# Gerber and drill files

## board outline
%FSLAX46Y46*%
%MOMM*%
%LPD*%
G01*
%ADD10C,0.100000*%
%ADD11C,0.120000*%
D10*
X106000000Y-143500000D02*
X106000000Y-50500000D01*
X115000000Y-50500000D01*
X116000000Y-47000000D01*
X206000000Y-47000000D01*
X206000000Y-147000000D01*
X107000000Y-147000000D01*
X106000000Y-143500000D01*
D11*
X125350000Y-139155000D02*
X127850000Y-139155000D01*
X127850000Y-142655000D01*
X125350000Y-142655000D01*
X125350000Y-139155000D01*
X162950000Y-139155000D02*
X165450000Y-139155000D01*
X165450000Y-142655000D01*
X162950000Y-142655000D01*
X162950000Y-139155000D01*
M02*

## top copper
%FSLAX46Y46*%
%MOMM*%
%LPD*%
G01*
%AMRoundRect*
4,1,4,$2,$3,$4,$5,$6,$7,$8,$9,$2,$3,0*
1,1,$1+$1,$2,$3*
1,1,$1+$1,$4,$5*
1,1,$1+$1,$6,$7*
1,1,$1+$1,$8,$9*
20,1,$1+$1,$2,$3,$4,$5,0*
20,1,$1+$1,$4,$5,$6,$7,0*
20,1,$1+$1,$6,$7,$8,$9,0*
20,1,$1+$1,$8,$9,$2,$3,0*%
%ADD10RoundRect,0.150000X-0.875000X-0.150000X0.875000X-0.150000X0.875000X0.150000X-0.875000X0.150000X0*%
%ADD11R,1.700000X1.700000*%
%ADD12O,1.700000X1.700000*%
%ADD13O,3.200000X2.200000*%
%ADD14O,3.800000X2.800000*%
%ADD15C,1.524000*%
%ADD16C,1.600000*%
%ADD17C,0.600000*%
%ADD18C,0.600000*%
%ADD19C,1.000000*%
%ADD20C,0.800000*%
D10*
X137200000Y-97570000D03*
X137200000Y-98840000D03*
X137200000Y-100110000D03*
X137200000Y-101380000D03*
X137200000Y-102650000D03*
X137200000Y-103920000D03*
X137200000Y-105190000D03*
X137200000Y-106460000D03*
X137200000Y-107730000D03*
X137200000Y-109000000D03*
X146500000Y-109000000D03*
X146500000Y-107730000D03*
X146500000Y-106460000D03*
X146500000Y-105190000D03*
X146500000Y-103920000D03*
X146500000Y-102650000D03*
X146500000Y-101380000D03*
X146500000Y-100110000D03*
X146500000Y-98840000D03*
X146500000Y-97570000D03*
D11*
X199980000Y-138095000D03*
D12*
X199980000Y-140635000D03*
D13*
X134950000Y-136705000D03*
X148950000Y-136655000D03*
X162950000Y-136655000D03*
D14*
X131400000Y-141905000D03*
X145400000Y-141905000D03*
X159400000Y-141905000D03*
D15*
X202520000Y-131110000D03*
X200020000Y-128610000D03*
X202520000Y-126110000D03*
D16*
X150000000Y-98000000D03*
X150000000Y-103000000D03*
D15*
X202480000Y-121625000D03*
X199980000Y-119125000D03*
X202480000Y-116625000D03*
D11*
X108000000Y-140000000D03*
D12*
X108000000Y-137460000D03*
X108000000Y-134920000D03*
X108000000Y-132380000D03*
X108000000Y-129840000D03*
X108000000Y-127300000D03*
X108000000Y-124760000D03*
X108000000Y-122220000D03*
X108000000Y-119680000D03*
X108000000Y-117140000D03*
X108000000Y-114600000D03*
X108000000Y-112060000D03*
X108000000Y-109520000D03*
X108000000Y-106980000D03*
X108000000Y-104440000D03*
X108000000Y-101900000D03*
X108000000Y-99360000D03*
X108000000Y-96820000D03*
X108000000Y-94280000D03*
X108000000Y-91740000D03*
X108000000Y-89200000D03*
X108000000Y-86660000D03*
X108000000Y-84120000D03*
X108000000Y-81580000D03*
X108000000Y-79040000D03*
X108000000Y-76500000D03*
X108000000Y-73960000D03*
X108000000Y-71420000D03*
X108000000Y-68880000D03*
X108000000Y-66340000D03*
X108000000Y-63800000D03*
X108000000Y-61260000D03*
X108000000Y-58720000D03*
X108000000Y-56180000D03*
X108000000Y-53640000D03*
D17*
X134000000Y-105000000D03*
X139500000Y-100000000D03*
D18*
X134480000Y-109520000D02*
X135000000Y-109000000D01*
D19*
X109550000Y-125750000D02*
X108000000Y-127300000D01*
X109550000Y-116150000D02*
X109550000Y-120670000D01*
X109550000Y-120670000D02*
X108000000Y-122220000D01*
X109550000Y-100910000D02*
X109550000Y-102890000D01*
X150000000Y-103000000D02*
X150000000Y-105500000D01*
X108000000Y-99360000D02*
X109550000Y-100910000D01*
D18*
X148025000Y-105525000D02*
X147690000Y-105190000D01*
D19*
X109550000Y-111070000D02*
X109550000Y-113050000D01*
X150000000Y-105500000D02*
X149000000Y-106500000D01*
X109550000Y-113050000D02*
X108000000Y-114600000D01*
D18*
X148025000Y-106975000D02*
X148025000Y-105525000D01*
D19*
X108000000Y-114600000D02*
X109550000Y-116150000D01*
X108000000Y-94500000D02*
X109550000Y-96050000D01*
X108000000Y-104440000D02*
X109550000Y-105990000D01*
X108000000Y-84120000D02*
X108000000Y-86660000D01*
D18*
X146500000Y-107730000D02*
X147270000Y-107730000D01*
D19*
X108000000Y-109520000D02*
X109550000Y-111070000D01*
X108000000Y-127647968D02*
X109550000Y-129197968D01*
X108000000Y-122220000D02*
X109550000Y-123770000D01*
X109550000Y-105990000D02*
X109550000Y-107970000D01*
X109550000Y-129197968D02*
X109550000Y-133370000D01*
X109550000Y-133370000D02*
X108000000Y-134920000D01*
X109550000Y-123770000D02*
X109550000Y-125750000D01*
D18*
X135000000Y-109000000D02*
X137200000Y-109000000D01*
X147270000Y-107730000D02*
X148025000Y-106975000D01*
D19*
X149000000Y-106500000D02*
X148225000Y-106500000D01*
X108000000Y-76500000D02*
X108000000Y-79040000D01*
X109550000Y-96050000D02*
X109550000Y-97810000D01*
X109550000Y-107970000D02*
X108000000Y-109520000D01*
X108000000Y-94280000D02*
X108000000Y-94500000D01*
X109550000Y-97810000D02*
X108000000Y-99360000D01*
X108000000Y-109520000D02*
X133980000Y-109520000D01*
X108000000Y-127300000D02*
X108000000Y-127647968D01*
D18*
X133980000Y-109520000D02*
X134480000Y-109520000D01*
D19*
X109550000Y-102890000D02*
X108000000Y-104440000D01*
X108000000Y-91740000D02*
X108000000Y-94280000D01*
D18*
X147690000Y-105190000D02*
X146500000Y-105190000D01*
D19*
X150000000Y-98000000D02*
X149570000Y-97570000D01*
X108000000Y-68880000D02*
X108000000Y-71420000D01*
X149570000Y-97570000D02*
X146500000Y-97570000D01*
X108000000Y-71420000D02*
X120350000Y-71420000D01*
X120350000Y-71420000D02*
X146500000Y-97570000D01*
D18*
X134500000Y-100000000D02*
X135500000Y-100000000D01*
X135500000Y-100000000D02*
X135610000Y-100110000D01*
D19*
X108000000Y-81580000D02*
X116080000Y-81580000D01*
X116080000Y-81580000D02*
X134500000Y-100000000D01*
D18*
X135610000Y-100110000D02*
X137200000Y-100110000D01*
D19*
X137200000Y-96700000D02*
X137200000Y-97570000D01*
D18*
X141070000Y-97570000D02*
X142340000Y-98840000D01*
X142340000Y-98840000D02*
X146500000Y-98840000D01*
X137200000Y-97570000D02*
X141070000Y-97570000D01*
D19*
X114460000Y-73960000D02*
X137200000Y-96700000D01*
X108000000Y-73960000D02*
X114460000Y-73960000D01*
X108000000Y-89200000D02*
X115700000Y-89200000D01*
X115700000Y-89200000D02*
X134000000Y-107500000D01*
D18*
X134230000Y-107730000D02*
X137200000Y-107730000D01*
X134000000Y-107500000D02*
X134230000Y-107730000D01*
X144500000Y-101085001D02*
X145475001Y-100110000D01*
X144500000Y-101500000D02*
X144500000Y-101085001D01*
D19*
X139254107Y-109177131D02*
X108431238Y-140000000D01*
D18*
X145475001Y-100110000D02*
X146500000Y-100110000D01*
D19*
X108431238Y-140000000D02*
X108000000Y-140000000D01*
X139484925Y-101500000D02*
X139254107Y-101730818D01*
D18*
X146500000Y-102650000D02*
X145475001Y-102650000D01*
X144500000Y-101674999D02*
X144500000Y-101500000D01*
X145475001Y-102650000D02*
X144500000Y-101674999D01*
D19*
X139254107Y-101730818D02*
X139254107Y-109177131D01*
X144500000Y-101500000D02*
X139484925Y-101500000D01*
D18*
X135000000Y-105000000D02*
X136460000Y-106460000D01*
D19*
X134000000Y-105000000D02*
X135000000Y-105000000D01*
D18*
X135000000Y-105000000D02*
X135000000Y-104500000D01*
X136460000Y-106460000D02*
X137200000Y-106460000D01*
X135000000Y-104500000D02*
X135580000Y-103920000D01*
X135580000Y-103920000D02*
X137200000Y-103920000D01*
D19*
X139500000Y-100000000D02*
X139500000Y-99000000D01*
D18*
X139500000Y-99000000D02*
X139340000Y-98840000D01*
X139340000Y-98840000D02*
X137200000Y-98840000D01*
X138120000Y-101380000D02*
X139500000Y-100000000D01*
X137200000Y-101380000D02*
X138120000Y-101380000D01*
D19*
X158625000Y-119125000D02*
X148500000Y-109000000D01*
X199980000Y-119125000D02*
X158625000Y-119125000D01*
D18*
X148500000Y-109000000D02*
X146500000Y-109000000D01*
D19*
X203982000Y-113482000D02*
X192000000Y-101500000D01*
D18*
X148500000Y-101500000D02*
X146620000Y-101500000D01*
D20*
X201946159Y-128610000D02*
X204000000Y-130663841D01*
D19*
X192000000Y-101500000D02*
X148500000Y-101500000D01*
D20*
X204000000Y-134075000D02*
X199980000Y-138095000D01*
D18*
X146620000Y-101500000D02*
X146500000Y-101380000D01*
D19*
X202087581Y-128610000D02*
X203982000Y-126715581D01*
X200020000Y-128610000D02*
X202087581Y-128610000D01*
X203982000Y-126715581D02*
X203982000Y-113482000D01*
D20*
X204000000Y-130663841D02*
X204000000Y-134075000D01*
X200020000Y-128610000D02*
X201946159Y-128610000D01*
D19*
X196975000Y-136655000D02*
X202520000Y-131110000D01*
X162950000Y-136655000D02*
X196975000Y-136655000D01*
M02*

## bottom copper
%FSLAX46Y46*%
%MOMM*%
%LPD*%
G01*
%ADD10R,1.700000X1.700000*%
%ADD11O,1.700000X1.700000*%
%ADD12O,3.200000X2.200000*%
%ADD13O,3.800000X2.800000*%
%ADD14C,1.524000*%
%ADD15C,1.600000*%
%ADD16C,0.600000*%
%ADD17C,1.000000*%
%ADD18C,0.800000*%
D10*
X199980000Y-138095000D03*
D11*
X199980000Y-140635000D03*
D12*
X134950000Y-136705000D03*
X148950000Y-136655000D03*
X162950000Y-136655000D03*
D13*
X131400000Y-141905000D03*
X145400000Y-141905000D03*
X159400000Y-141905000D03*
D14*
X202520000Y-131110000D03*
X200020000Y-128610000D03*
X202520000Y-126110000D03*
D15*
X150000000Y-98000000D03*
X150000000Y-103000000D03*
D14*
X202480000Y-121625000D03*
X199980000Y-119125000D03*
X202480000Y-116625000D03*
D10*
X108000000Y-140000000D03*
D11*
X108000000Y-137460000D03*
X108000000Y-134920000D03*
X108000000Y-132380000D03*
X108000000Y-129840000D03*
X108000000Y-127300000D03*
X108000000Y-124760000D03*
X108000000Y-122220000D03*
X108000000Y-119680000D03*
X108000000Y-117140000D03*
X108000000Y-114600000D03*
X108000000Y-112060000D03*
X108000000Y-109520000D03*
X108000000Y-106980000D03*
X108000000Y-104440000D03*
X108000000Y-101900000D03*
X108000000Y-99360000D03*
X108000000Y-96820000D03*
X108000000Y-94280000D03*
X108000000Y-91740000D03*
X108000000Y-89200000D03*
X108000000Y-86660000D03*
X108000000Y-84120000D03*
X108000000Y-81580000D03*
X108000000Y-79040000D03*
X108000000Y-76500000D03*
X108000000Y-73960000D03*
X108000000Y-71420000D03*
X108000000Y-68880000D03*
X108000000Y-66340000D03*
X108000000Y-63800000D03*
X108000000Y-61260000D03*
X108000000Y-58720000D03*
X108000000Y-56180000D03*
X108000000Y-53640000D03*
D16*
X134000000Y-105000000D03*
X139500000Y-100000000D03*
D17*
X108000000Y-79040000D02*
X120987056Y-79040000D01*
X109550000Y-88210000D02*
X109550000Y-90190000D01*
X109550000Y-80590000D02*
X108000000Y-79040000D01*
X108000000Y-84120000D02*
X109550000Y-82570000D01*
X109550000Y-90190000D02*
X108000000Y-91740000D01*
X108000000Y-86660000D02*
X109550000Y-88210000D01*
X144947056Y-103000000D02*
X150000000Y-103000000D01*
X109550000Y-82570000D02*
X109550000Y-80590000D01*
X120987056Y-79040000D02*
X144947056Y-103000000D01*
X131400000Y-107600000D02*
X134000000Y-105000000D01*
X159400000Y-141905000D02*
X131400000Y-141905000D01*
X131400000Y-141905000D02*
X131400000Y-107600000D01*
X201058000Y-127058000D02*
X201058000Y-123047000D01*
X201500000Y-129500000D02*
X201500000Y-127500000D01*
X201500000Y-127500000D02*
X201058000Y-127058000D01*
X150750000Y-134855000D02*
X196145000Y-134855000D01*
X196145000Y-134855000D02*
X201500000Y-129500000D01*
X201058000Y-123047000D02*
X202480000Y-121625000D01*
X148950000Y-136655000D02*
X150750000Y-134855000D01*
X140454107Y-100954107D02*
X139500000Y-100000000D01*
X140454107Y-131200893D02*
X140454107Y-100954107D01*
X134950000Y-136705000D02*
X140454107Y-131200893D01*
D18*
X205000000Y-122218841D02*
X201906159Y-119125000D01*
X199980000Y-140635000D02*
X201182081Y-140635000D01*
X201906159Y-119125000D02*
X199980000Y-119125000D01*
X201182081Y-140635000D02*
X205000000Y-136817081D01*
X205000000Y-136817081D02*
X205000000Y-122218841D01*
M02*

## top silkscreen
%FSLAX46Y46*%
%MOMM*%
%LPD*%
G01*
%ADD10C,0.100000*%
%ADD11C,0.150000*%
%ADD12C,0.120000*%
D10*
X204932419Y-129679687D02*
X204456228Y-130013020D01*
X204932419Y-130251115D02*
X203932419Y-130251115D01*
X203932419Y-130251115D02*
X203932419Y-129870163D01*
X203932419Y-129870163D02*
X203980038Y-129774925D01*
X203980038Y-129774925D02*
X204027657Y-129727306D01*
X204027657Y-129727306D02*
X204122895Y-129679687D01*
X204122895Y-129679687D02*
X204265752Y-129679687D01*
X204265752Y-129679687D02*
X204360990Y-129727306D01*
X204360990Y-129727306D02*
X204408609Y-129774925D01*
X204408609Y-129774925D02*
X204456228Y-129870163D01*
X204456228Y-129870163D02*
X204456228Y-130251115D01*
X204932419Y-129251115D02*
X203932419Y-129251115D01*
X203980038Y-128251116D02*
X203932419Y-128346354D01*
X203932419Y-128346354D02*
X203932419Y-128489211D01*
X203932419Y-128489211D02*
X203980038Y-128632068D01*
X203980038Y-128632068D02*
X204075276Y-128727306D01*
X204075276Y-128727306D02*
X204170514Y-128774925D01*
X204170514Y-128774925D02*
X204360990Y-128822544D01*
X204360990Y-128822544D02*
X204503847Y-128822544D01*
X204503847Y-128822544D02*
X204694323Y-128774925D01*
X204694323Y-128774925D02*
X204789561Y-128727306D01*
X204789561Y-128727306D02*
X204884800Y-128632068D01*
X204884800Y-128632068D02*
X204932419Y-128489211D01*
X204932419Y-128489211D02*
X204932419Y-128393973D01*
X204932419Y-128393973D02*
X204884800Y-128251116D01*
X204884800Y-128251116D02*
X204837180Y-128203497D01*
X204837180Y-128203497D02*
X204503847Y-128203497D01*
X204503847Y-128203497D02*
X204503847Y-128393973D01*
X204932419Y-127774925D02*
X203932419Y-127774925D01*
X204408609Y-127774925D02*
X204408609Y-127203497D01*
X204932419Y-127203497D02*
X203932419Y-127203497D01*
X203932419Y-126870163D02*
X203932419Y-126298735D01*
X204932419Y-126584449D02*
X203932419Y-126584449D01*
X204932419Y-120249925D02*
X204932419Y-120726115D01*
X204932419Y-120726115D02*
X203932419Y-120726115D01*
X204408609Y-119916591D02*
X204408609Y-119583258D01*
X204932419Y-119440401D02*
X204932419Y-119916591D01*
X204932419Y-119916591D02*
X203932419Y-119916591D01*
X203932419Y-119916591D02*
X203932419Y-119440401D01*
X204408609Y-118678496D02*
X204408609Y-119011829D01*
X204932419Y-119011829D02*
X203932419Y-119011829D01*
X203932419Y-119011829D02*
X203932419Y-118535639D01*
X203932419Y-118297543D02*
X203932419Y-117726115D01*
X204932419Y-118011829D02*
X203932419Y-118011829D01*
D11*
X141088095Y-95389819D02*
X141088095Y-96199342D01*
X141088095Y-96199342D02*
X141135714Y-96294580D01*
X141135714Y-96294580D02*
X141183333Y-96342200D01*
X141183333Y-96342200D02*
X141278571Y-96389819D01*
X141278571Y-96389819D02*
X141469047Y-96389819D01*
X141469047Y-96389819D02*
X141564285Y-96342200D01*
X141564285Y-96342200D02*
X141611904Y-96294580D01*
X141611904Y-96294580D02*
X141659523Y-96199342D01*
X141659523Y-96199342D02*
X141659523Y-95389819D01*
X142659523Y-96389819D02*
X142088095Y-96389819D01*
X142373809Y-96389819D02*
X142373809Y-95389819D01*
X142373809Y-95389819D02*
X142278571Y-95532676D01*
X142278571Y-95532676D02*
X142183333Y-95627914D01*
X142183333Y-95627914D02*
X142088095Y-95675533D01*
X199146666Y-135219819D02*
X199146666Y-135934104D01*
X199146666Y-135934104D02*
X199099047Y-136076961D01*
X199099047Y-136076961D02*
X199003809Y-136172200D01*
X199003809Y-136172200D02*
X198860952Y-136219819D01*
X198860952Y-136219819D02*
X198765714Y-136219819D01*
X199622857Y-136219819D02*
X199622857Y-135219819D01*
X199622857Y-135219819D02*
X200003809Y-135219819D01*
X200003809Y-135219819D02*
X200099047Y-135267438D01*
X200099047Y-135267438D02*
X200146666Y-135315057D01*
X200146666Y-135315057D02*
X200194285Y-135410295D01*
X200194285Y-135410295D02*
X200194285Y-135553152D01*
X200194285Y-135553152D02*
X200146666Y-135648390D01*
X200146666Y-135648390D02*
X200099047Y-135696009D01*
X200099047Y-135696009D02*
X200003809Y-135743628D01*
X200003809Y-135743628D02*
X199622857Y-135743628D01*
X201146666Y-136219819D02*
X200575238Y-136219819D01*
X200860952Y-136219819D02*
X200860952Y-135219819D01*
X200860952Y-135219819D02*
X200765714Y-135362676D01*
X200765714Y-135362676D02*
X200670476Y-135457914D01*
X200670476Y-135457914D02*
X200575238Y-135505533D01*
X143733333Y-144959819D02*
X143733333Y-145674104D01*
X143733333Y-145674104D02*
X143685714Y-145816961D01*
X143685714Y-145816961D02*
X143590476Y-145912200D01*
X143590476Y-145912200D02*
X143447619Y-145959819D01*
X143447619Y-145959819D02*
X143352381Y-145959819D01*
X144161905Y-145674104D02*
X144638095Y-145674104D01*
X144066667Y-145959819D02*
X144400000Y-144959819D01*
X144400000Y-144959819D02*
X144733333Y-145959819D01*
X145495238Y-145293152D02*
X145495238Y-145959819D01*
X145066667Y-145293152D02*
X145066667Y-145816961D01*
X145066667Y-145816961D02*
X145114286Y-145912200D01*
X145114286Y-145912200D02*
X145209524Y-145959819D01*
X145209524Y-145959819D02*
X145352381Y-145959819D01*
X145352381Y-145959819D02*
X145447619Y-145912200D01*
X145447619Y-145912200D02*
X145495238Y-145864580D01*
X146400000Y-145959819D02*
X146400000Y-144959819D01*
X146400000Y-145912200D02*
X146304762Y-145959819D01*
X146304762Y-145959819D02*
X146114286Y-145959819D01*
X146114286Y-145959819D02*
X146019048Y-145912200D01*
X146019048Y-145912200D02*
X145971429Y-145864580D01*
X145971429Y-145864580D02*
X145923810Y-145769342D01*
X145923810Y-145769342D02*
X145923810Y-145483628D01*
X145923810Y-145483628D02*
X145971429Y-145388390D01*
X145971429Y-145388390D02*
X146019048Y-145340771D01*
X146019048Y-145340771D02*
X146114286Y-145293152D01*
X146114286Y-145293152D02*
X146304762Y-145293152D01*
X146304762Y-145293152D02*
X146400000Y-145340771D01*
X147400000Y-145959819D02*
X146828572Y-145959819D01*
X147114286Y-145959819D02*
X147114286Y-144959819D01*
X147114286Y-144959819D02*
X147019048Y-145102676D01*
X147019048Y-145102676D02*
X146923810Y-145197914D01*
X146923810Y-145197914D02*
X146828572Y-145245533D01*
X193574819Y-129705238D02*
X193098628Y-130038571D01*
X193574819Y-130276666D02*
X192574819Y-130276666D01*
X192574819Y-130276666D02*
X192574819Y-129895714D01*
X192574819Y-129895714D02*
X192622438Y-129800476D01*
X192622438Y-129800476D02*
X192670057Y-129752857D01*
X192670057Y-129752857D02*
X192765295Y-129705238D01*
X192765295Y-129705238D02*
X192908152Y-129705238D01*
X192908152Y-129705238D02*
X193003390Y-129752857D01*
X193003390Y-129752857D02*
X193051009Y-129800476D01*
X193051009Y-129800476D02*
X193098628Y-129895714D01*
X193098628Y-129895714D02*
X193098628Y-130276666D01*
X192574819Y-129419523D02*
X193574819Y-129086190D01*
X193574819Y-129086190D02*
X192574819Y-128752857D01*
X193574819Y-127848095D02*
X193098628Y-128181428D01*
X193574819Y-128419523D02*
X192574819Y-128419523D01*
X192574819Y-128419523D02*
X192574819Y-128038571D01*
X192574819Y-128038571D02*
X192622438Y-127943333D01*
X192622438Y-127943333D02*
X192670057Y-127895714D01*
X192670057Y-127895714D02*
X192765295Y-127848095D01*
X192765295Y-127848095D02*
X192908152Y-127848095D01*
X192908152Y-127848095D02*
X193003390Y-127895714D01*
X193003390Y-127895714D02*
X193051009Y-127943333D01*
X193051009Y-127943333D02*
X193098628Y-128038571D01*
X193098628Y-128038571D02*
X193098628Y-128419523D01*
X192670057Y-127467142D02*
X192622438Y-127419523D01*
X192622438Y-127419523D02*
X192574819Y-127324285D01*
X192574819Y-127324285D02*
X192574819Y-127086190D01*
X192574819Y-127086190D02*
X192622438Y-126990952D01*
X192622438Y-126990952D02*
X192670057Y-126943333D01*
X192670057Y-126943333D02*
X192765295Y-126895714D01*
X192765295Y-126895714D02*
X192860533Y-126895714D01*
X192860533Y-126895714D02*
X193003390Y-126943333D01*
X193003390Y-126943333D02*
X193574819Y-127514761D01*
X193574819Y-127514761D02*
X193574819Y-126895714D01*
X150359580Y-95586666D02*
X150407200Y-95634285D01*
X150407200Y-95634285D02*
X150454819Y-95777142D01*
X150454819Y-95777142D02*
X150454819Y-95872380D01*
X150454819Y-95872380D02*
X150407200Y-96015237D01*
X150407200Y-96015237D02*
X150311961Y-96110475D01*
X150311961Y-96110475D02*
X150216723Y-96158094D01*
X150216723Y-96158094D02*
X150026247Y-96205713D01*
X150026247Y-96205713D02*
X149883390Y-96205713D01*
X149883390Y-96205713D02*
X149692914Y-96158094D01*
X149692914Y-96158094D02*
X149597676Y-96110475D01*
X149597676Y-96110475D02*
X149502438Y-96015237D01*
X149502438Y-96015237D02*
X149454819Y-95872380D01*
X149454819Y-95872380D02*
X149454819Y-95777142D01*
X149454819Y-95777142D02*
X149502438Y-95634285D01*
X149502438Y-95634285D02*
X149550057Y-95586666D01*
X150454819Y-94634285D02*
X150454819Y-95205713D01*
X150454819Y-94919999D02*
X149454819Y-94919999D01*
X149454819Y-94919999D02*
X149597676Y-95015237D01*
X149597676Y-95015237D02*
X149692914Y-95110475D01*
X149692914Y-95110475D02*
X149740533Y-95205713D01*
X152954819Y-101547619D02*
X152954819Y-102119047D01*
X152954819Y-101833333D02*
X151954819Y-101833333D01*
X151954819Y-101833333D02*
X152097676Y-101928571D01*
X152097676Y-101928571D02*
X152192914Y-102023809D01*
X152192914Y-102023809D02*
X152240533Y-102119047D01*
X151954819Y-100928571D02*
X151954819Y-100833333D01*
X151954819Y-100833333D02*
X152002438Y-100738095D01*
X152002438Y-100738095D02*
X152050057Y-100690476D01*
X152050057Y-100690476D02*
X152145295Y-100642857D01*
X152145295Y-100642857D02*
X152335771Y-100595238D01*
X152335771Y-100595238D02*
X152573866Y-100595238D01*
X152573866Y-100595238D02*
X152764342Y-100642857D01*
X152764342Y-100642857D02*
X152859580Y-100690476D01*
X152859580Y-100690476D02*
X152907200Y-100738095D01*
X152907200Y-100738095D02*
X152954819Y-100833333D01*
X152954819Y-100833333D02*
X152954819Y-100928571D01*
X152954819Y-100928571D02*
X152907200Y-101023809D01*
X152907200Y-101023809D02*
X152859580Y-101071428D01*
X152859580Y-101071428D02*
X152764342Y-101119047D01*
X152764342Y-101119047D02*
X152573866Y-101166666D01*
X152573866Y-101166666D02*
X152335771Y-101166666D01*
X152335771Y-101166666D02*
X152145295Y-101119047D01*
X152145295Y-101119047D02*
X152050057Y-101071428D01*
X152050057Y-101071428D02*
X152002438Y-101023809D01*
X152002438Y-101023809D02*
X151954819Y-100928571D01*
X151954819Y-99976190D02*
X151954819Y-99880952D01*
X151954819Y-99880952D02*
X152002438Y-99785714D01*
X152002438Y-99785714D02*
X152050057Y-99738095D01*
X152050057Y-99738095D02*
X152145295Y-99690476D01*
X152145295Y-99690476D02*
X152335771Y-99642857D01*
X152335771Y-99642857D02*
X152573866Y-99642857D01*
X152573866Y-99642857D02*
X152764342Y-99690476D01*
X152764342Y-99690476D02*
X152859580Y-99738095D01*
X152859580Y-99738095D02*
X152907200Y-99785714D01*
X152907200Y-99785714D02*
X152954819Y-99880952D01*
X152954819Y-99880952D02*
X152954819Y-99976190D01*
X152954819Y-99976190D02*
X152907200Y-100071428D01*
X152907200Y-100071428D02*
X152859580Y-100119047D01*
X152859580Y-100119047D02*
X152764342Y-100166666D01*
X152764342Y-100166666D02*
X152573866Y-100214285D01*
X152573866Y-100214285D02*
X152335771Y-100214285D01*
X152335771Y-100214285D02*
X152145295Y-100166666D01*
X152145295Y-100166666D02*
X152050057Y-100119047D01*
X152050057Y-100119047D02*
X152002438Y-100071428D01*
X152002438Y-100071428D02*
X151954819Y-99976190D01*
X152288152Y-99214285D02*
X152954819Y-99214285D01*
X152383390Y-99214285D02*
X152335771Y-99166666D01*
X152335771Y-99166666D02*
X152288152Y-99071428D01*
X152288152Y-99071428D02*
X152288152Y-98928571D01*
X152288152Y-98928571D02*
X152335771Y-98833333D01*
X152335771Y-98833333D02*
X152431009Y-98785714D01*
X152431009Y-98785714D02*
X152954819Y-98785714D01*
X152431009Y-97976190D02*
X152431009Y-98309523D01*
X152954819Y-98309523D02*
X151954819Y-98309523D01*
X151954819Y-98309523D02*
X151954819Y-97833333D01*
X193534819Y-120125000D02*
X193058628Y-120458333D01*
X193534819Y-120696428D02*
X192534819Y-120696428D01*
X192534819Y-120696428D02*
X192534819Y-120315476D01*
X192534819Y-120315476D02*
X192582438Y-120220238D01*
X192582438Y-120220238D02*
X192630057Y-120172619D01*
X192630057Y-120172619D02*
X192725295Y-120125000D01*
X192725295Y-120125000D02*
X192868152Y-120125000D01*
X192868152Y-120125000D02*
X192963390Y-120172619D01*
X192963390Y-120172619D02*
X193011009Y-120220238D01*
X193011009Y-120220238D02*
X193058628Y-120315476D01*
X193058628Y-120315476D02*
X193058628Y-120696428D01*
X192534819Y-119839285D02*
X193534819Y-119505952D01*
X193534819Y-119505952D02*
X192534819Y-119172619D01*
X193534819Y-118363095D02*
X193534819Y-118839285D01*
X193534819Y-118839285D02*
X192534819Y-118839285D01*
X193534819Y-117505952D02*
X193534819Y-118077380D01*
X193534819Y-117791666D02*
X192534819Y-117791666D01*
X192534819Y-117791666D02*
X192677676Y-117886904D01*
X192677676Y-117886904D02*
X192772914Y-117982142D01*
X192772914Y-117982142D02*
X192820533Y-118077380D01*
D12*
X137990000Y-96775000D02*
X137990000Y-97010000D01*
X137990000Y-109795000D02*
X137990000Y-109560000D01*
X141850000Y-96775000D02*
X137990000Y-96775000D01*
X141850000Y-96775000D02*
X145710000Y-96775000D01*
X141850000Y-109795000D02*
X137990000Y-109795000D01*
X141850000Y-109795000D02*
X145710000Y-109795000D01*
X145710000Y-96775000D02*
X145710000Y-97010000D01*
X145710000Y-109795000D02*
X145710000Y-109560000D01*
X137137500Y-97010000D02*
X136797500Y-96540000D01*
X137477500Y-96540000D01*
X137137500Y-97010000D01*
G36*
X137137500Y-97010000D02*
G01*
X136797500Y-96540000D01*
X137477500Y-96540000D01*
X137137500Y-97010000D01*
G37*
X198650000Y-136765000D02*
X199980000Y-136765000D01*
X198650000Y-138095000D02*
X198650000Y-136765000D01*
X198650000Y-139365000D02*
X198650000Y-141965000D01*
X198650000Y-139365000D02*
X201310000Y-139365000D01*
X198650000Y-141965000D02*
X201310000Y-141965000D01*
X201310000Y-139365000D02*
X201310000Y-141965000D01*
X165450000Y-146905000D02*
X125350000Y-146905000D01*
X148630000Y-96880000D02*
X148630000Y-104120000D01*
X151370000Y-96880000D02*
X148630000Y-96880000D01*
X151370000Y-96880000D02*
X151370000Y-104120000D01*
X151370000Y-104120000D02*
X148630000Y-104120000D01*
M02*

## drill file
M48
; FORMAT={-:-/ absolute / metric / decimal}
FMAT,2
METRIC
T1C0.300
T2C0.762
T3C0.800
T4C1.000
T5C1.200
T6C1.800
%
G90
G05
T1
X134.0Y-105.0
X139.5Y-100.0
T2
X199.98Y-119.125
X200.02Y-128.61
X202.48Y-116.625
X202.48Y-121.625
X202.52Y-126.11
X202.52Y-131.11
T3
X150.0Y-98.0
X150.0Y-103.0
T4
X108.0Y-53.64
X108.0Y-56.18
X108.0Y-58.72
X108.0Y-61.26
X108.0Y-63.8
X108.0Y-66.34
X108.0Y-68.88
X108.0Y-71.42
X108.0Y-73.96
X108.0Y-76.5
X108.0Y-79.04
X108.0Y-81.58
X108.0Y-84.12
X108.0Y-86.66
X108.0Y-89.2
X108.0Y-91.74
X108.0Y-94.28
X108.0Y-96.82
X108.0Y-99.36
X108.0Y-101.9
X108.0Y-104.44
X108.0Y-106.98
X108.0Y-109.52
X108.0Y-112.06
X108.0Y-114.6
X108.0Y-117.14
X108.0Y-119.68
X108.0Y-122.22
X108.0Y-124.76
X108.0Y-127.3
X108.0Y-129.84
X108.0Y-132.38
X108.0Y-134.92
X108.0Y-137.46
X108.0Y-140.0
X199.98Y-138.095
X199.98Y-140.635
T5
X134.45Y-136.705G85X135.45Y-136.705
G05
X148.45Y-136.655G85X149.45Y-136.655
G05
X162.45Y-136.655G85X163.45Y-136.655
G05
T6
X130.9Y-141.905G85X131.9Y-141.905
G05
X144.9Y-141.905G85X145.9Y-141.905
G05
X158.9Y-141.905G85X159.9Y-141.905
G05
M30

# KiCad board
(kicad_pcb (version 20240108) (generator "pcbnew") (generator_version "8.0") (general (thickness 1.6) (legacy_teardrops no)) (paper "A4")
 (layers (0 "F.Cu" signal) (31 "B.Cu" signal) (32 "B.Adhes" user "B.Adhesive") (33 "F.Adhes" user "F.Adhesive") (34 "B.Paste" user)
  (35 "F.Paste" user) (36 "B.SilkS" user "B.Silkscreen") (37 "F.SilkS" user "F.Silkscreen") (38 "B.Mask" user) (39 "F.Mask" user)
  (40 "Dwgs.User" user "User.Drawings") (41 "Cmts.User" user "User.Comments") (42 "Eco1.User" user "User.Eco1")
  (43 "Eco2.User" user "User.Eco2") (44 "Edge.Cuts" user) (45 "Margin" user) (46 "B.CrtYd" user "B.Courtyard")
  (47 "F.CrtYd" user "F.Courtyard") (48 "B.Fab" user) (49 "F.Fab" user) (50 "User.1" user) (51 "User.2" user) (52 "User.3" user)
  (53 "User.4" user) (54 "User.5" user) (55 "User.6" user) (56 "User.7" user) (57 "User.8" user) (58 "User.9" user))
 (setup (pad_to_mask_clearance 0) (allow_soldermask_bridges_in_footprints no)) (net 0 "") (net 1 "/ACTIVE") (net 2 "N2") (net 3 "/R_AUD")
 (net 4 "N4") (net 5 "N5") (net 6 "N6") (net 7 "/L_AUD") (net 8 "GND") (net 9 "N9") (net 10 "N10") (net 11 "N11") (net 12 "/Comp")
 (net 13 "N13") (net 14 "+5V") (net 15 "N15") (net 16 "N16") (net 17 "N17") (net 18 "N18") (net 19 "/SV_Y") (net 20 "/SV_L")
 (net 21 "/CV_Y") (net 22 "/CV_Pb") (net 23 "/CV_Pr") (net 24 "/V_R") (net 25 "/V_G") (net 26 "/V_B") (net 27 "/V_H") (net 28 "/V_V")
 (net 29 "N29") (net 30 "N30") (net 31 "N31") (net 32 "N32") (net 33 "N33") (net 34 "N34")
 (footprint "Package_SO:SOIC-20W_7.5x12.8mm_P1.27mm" (layer "F.Cu") (at 141.85 103.285)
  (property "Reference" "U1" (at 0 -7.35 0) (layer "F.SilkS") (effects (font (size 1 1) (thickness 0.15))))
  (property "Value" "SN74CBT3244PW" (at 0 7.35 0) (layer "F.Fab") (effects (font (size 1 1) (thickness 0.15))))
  (fp_line (start -3.86 -6.51) (end -3.86 -6.275) (stroke (width 0.12) (type solid)) (layer "F.SilkS"))
  (fp_line (start -3.86 6.51) (end -3.86 6.275) (stroke (width 0.12) (type solid)) (layer "F.SilkS"))
  (fp_line (start 0 -6.51) (end -3.86 -6.51) (stroke (width 0.12) (type solid)) (layer "F.SilkS"))
  (fp_line (start 0 -6.51) (end 3.86 -6.51) (stroke (width 0.12) (type solid)) (layer "F.SilkS"))
  (fp_line (start 0 6.51) (end -3.86 6.51) (stroke (width 0.12) (type solid)) (layer "F.SilkS"))
  (fp_line (start 0 6.51) (end 3.86 6.51) (stroke (width 0.12) (type solid)) (layer "F.SilkS"))
  (fp_line (start 3.86 -6.51) (end 3.86 -6.275) (stroke (width 0.12) (type solid)) (layer "F.SilkS"))
  (fp_line (start 3.86 6.51) (end 3.86 6.275) (stroke (width 0.12) (type solid)) (layer "F.SilkS"))
  (fp_poly
   (pts (xy -4.7125 -6.275) (xy -5.0525 -6.745) (xy -4.3725 -6.745) (xy -4.7125 -6.275)) (stroke (width 0.12) (type solid)) (fill solid)
   (layer "F.SilkS"))
  (pad "1" smd roundrect (at -4.65 -5.715) (size 2.05 0.6) (layers "F.Cu" "F.Paste" "F.Mask") (roundrect_rratio 0.25) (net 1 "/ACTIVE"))
  (pad "2" smd roundrect (at -4.65 -4.445) (size 2.05 0.6) (layers "F.Cu" "F.Paste" "F.Mask") (roundrect_rratio 0.25) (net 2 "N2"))
  (pad "3" smd roundrect (at -4.65 -3.175) (size 2.05 0.6) (layers "F.Cu" "F.Paste" "F.Mask") (roundrect_rratio 0.25) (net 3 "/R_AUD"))
  (pad "4" smd roundrect (at -4.65 -1.905) (size 2.05 0.6) (layers "F.Cu" "F.Paste" "F.Mask") (roundrect_rratio 0.25) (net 2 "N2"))
  (pad "5" smd roundrect (at -4.65 -0.635) (size 2.05 0.6) (layers "F.Cu" "F.Paste" "F.Mask") (roundrect_rratio 0.25) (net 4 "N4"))
  (pad "6" smd roundrect (at -4.65 0.635) (size 2.05 0.6) (layers "F.Cu" "F.Paste" "F.Mask") (roundrect_rratio 0.25) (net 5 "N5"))
  (pad "7" smd roundrect (at -4.65 1.905) (size 2.05 0.6) (layers "F.Cu" "F.Paste" "F.Mask") (roundrect_rratio 0.25) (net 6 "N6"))
  (pad "8" smd roundrect (at -4.65 3.175) (size 2.05 0.6) (layers "F.Cu" "F.Paste" "F.Mask") (roundrect_rratio 0.25) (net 5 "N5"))
  (pad "9" smd roundrect (at -4.65 4.445) (size 2.05 0.6) (layers "F.Cu" "F.Paste" "F.Mask") (roundrect_rratio 0.25) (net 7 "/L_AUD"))
  (pad "10" smd roundrect (at -4.65 5.715) (size 2.05 0.6) (layers "F.Cu" "F.Paste" "F.Mask") (roundrect_rratio 0.25) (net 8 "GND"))
  (pad "11" smd roundrect (at 4.65 5.715) (size 2.05 0.6) (layers "F.Cu" "F.Paste" "F.Mask") (roundrect_rratio 0.25) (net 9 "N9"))
  (pad "12" smd roundrect (at 4.65 4.445) (size 2.05 0.6) (layers "F.Cu" "F.Paste" "F.Mask") (roundrect_rratio 0.25) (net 8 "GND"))
  (pad "13" smd roundrect (at 4.65 3.175) (size 2.05 0.6) (layers "F.Cu" "F.Paste" "F.Mask") (roundrect_rratio 0.25) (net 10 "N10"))
  (pad "14" smd roundrect (at 4.65 1.905) (size 2.05 0.6) (layers "F.Cu" "F.Paste" "F.Mask") (roundrect_rratio 0.25) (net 8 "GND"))
  (pad "15" smd roundrect (at 4.65 0.635) (size 2.05 0.6) (layers "F.Cu" "F.Paste" "F.Mask") (roundrect_rratio 0.25) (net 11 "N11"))
  (pad "16" smd roundrect (at 4.65 -0.635) (size 2.05 0.6) (layers "F.Cu" "F.Paste" "F.Mask") (roundrect_rratio 0.25) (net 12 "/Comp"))
  (pad "17" smd roundrect (at 4.65 -1.905) (size 2.05 0.6) (layers "F.Cu" "F.Paste" "F.Mask") (roundrect_rratio 0.25) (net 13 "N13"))
  (pad "18" smd roundrect (at 4.65 -3.175) (size 2.05 0.6) (layers "F.Cu" "F.Paste" "F.Mask") (roundrect_rratio 0.25) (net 12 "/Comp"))
  (pad "19" smd roundrect (at 4.65 -4.445) (size 2.05 0.6) (layers "F.Cu" "F.Paste" "F.Mask") (roundrect_rratio 0.25) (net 1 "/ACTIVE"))
  (pad "20" smd roundrect (at 4.65 -5.715) (size 2.05 0.6) (layers "F.Cu" "F.Paste" "F.Mask") (roundrect_rratio 0.25) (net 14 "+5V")))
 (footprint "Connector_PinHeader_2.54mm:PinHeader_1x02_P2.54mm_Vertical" (layer "F.Cu") (at 199.98 138.095)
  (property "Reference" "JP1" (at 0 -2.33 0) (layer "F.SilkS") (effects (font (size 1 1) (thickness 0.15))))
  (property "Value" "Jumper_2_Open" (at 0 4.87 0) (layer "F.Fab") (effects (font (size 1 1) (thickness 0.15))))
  (fp_line (start -1.33 -1.33) (end 0 -1.33) (stroke (width 0.12) (type solid)) (layer "F.SilkS"))
  (fp_line (start -1.33 0) (end -1.33 -1.33) (stroke (width 0.12) (type solid)) (layer "F.SilkS"))
  (fp_line (start -1.33 1.27) (end -1.33 3.87) (stroke (width 0.12) (type solid)) (layer "F.SilkS"))
  (fp_line (start -1.33 1.27) (end 1.33 1.27) (stroke (width 0.12) (type solid)) (layer "F.SilkS"))
  (fp_line (start -1.33 3.87) (end 1.33 3.87) (stroke (width 0.12) (type solid)) (layer "F.SilkS"))
  (fp_line (start 1.33 1.27) (end 1.33 3.87) (stroke (width 0.12) (type solid)) (layer "F.SilkS"))
  (pad "1" thru_hole rect (at 0 0) (size 1.7 1.7) (drill 1) (layers "*.Cu" "*.Mask") (remove_unused_layers no) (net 13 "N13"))
  (pad "2" thru_hole oval (at 0 2.54) (size 1.7 1.7) (drill 1) (layers "*.Cu" "*.Mask") (remove_unused_layers no) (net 9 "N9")))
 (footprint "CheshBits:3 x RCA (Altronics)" (layer "F.Cu") (at 145.4 146.905)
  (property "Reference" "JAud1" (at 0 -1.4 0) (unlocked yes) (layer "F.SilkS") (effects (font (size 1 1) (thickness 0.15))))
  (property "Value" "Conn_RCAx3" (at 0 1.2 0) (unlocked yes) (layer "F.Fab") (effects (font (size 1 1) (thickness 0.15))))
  (fp_line (start 20.05 0) (end -20.05 0) (stroke (width 0.12) (type default)) (layer "F.SilkS"))
  (fp_rect (start -20.05 -7.75) (end -17.55 -4.25) (stroke (width 0.12) (type default)) (fill none) (layer "Edge.Cuts"))
  (fp_rect (start 17.55 -7.75) (end 20.05 -4.25) (stroke (width 0.12) (type default)) (fill none) (layer "Edge.Cuts"))
  (pad "1" thru_hole oval (at -10.45 -10.2) (size 3.2 2.2) (drill oval 2.2 1.2) (layers "*.Cu" "*.Mask") (remove_unused_layers no)
   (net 2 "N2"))
  (pad "2" thru_hole oval (at 3.55 -10.25) (size 3.2 2.2) (drill oval 2.2 1.2) (layers "*.Cu" "*.Mask") (remove_unused_layers no)
   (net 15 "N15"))
  (pad "3" thru_hole oval (at 17.55 -10.25) (size 3.2 2.2) (drill oval 2.2 1.2) (layers "*.Cu" "*.Mask") (remove_unused_layers no)
   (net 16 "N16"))
  (pad "4" thru_hole oval (at -14 -5) (size 3.8 2.8) (drill oval 2.8 1.8) (layers "*.Cu" "*.Mask") (remove_unused_layers no) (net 5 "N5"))
  (pad "4" thru_hole oval (at 0 -5) (size 3.8 2.8) (drill oval 2.8 1.8) (layers "*.Cu" "*.Mask") (remove_unused_layers no) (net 5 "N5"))
  (pad "4" thru_hole oval (at 14 -5) (size 3.8 2.8) (drill oval 2.8 1.8) (layers "*.Cu" "*.Mask") (remove_unused_layers no) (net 5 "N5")))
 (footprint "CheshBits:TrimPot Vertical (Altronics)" (layer "F.Cu") (at 193.62 128.61 90)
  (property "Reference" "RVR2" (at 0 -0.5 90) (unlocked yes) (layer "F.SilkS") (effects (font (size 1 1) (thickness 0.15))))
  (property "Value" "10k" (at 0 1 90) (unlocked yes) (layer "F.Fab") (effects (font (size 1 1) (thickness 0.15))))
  (pad "1" thru_hole circle (at -2.5 8.9 90) (size 1.524 1.524) (drill 0.762) (layers "*.Cu" "*.Mask") (remove_unused_layers no)
   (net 16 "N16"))
  (pad "2" thru_hole circle (at 0 6.4 90) (size 1.524 1.524) (drill 0.762) (layers "*.Cu" "*.Mask") (remove_unused_layers no) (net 13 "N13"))
  (pad "3" thru_hole circle (at 2.5 8.9 90) (size 1.524 1.524) (drill 0.762) (layers "*.Cu" "*.Mask") (remove_unused_layers no)
   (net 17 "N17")))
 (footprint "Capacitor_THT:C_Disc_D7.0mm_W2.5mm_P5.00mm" (layer "F.Cu") (at 150 98 -90)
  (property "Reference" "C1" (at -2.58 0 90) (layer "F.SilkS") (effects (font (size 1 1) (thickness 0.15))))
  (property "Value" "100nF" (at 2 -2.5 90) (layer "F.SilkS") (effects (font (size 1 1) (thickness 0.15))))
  (fp_line (start -1.12 1.37) (end 6.12 1.37) (stroke (width 0.12) (type solid)) (layer "F.SilkS"))
  (fp_line (start -1.12 -1.37) (end -1.12 1.37) (stroke (width 0.12) (type solid)) (layer "F.SilkS"))
  (fp_line (start -1.12 -1.37) (end 6.12 -1.37) (stroke (width 0.12) (type solid)) (layer "F.SilkS"))
  (fp_line (start 6.12 -1.37) (end 6.12 1.37) (stroke (width 0.12) (type solid)) (layer "F.SilkS"))
  (pad "1" thru_hole circle (at 0 0 270) (size 1.6 1.6) (drill 0.8) (layers "*.Cu" "*.Mask") (remove_unused_layers no) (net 14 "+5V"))
  (pad "2" thru_hole circle (at 5 0 270) (size 1.6 1.6) (drill 0.8) (layers "*.Cu" "*.Mask") (remove_unused_layers no) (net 8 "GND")))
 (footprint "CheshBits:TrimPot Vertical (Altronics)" (layer "F.Cu") (at 193.58 119.125 90)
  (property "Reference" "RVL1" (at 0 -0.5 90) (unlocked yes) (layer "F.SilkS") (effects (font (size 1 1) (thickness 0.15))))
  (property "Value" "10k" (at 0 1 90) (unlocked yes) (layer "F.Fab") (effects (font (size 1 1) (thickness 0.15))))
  (pad "1" thru_hole circle (at -2.5 8.9 90) (size 1.524 1.524) (drill 0.762) (layers "*.Cu" "*.Mask") (remove_unused_layers no)
   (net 15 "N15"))
  (pad "2" thru_hole circle (at 0 6.4 90) (size 1.524 1.524) (drill 0.762) (layers "*.Cu" "*.Mask") (remove_unused_layers no) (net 9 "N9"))
  (pad "3" thru_hole circle (at 2.5 8.9 90) (size 1.524 1.524) (drill 0.762) (layers "*.Cu" "*.Mask") (remove_unused_layers no)
   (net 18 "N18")))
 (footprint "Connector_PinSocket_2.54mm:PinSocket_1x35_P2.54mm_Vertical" (layer "B.Cu") (at 108 140)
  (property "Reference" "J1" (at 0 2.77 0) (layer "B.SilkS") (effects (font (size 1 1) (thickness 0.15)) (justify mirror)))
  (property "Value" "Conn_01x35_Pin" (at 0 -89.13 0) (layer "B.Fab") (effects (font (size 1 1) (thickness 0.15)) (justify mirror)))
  (pad "1" thru_hole rect (at 0 0) (size 1.7 1.7) (drill 1) (layers "*.Cu" "*.Mask") (remove_unused_layers no) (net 12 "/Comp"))
  (pad "2" thru_hole oval (at 0 -2.54) (size 1.7 1.7) (drill 1) (layers "*.Cu" "*.Mask") (remove_unused_layers no) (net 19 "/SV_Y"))
  (pad "3" thru_hole oval (at 0 -5.08) (size 1.7 1.7) (drill 1) (layers "*.Cu" "*.Mask") (remove_unused_layers no) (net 8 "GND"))
  (pad "4" thru_hole oval (at 0 -7.62) (size 1.7 1.7) (drill 1) (layers "*.Cu" "*.Mask") (remove_unused_layers no) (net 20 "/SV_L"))
  (pad "5" thru_hole oval (at 0 -10.16) (size 1.7 1.7) (drill 1) (layers "*.Cu" "*.Mask") (remove_unused_layers no) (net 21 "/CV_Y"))
  (pad "6" thru_hole oval (at 0 -12.7) (size 1.7 1.7) (drill 1) (layers "*.Cu" "*.Mask") (remove_unused_layers no) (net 8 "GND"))
  (pad "7" thru_hole oval (at 0 -15.24) (size 1.7 1.7) (drill 1) (layers "*.Cu" "*.Mask") (remove_unused_layers no) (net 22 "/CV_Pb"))
  (pad "8" thru_hole oval (at 0 -17.78) (size 1.7 1.7) (drill 1) (layers "*.Cu" "*.Mask") (remove_unused_layers no) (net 8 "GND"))
  (pad "9" thru_hole oval (at 0 -20.32) (size 1.7 1.7) (drill 1) (layers "*.Cu" "*.Mask") (remove_unused_layers no) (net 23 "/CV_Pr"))
  (pad "10" thru_hole oval (at 0 -22.86) (size 1.7 1.7) (drill 1) (layers "*.Cu" "*.Mask") (remove_unused_layers no) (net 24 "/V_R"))
  (pad "11" thru_hole oval (at 0 -25.4) (size 1.7 1.7) (drill 1) (layers "*.Cu" "*.Mask") (remove_unused_layers no) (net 8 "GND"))
  (pad "12" thru_hole oval (at 0 -27.94) (size 1.7 1.7) (drill 1) (layers "*.Cu" "*.Mask") (remove_unused_layers no) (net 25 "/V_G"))
  (pad "13" thru_hole oval (at 0 -30.48) (size 1.7 1.7) (drill 1) (layers "*.Cu" "*.Mask") (remove_unused_layers no) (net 8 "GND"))
  (pad "14" thru_hole oval (at 0 -33.02) (size 1.7 1.7) (drill 1) (layers "*.Cu" "*.Mask") (remove_unused_layers no) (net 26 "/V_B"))
  (pad "15" thru_hole oval (at 0 -35.56) (size 1.7 1.7) (drill 1) (layers "*.Cu" "*.Mask") (remove_unused_layers no) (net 8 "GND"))
  (pad "16" thru_hole oval (at 0 -38.1) (size 1.7 1.7) (drill 1) (layers "*.Cu" "*.Mask") (remove_unused_layers no) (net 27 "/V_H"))
  (pad "17" thru_hole oval (at 0 -40.64) (size 1.7 1.7) (drill 1) (layers "*.Cu" "*.Mask") (remove_unused_layers no) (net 8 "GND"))
  (pad "18" thru_hole oval (at 0 -43.18) (size 1.7 1.7) (drill 1) (layers "*.Cu" "*.Mask") (remove_unused_layers no) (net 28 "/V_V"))
  (pad "19" thru_hole oval (at 0 -45.72) (size 1.7 1.7) (drill 1) (layers "*.Cu" "*.Mask") (remove_unused_layers no) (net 8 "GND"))
  (pad "20" thru_hole oval (at 0 -48.26) (size 1.7 1.7) (drill 1) (layers "*.Cu" "*.Mask") (remove_unused_layers no) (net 8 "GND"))
  (pad "21" thru_hole oval (at 0 -50.8) (size 1.7 1.7) (drill 1) (layers "*.Cu" "*.Mask") (remove_unused_layers no) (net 7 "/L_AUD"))
  (pad "22" thru_hole oval (at 0 -53.34) (size 1.7 1.7) (drill 1) (layers "*.Cu" "*.Mask") (remove_unused_layers no) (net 8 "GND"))
  (pad "23" thru_hole oval (at 0 -55.88) (size 1.7 1.7) (drill 1) (layers "*.Cu" "*.Mask") (remove_unused_layers no) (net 8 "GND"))
  (pad "24" thru_hole oval (at 0 -58.42) (size 1.7 1.7) (drill 1) (layers "*.Cu" "*.Mask") (remove_unused_layers no) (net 3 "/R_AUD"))
  (pad "25" thru_hole oval (at 0 -60.96) (size 1.7 1.7) (drill 1) (layers "*.Cu" "*.Mask") (remove_unused_layers no) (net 8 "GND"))
  (pad "26" thru_hole oval (at 0 -63.5) (size 1.7 1.7) (drill 1) (layers "*.Cu" "*.Mask") (remove_unused_layers no) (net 8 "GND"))
  (pad "27" thru_hole oval (at 0 -66.04) (size 1.7 1.7) (drill 1) (layers "*.Cu" "*.Mask") (remove_unused_layers no) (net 1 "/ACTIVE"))
  (pad "28" thru_hole oval (at 0 -68.58) (size 1.7 1.7) (drill 1) (layers "*.Cu" "*.Mask") (remove_unused_layers no) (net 14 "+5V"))
  (pad "29" thru_hole oval (at 0 -71.12) (size 1.7 1.7) (drill 1) (layers "*.Cu" "*.Mask") (remove_unused_layers no) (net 14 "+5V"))
  (pad "30" thru_hole oval (at 0 -73.66) (size 1.7 1.7) (drill 1) (layers "*.Cu" "*.Mask") (remove_unused_layers no) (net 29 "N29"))
  (pad "31" thru_hole oval (at 0 -76.2) (size 1.7 1.7) (drill 1) (layers "*.Cu" "*.Mask") (remove_unused_layers no) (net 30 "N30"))
  (pad "32" thru_hole oval (at 0 -78.74) (size 1.7 1.7) (drill 1) (layers "*.Cu" "*.Mask") (remove_unused_layers no) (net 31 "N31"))
  (pad "33" thru_hole oval (at 0 -81.28) (size 1.7 1.7) (drill 1) (layers "*.Cu" "*.Mask") (remove_unused_layers no) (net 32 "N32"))
  (pad "34" thru_hole oval (at 0 -83.82) (size 1.7 1.7) (drill 1) (layers "*.Cu" "*.Mask") (remove_unused_layers no) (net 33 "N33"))
  (pad "35" thru_hole oval (at 0 -86.36) (size 1.7 1.7) (drill 1) (layers "*.Cu" "*.Mask") (remove_unused_layers no) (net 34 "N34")))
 (gr_poly
  (pts (xy 106 143.5) (xy 106 50.5) (xy 115 50.5) (xy 116 47) (xy 206 47) (xy 206 147) (xy 107 147)) (stroke (width 0.1) (type solid))
  (fill none) (layer "Edge.Cuts"))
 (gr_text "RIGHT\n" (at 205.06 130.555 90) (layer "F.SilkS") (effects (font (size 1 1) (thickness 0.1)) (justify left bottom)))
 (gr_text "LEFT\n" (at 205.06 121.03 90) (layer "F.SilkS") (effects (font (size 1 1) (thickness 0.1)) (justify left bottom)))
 (segment (start 134.48 109.52) (end 135 109) (width 0.6) (layer "F.Cu") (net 8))
 (segment (start 109.55 125.75) (end 108 127.3) (width 1) (layer "F.Cu") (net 8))
 (segment (start 109.55 116.15) (end 109.55 120.67) (width 1) (layer "F.Cu") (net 8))
 (segment (start 109.55 120.67) (end 108 122.22) (width 1) (layer "F.Cu") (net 8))
 (segment (start 109.55 100.91) (end 109.55 102.89) (width 1) (layer "F.Cu") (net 8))
 (segment (start 150 103) (end 150 105.5) (width 1) (layer "F.Cu") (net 8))
 (segment (start 108 99.36) (end 109.55 100.91) (width 1) (layer "F.Cu") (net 8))
 (segment (start 148.025 105.525) (end 147.69 105.19) (width 0.6) (layer "F.Cu") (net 8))
 (segment (start 109.55 111.07) (end 109.55 113.05) (width 1) (layer "F.Cu") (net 8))
 (segment (start 150 105.5) (end 149 106.5) (width 1) (layer "F.Cu") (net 8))
 (segment (start 109.55 113.05) (end 108 114.6) (width 1) (layer "F.Cu") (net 8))
 (segment (start 148.025 106.975) (end 148.025 105.525) (width 0.6) (layer "F.Cu") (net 8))
 (segment (start 108 114.6) (end 109.55 116.15) (width 1) (layer "F.Cu") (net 8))
 (segment (start 108 94.5) (end 109.55 96.05) (width 1) (layer "F.Cu") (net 8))
 (segment (start 108 104.44) (end 109.55 105.99) (width 1) (layer "F.Cu") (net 8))
 (segment (start 108 84.12) (end 108 86.66) (width 1) (layer "F.Cu") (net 8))
 (segment (start 146.5 107.73) (end 147.27 107.73) (width 0.6) (layer "F.Cu") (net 8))
 (segment (start 108 109.52) (end 109.55 111.07) (width 1) (layer "F.Cu") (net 8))
 (segment (start 108 127.647968) (end 109.55 129.197968) (width 1) (layer "F.Cu") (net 8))
 (segment (start 108 122.22) (end 109.55 123.77) (width 1) (layer "F.Cu") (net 8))
 (segment (start 109.55 105.99) (end 109.55 107.97) (width 1) (layer "F.Cu") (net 8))
 (segment (start 109.55 129.197968) (end 109.55 133.37) (width 1) (layer "F.Cu") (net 8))
 (segment (start 109.55 133.37) (end 108 134.92) (width 1) (layer "F.Cu") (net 8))
 (segment (start 109.55 123.77) (end 109.55 125.75) (width 1) (layer "F.Cu") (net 8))
 (segment (start 135 109) (end 137.2 109) (width 0.6) (layer "F.Cu") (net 8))
 (segment (start 147.27 107.73) (end 148.025 106.975) (width 0.6) (layer "F.Cu") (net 8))
 (segment (start 149 106.5) (end 148.225 106.5) (width 1) (layer "F.Cu") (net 8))
 (segment (start 108 76.5) (end 108 79.04) (width 1) (layer "F.Cu") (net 8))
 (segment (start 109.55 96.05) (end 109.55 97.81) (width 1) (layer "F.Cu") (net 8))
 (segment (start 109.55 107.97) (end 108 109.52) (width 1) (layer "F.Cu") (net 8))
 (segment (start 108 94.28) (end 108 94.5) (width 1) (layer "F.Cu") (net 8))
 (segment (start 109.55 97.81) (end 108 99.36) (width 1) (layer "F.Cu") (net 8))
 (segment (start 108 109.52) (end 133.98 109.52) (width 1) (layer "F.Cu") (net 8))
 (segment (start 108 127.3) (end 108 127.647968) (width 1) (layer "F.Cu") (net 8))
 (segment (start 133.98 109.52) (end 134.48 109.52) (width 0.6) (layer "F.Cu") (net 8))
 (segment (start 109.55 102.89) (end 108 104.44) (width 1) (layer "F.Cu") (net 8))
 (segment (start 108 91.74) (end 108 94.28) (width 1) (layer "F.Cu") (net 8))
 (segment (start 147.69 105.19) (end 146.5 105.19) (width 0.6) (layer "F.Cu") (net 8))
 (segment (start 108 79.04) (end 120.987056 79.04) (width 1) (layer "B.Cu") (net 8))
 (segment (start 109.55 88.21) (end 109.55 90.19) (width 1) (layer "B.Cu") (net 8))
 (segment (start 109.55 80.59) (end 108 79.04) (width 1) (layer "B.Cu") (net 8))
 (segment (start 108 84.12) (end 109.55 82.57) (width 1) (layer "B.Cu") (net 8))
 (segment (start 109.55 90.19) (end 108 91.74) (width 1) (layer "B.Cu") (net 8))
 (segment (start 108 86.66) (end 109.55 88.21) (width 1) (layer "B.Cu") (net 8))
 (segment (start 144.947056 103) (end 150 103) (width 1) (layer "B.Cu") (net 8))
 (segment (start 109.55 82.57) (end 109.55 80.59) (width 1) (layer "B.Cu") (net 8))
 (segment (start 120.987056 79.04) (end 144.947056 103) (width 1) (layer "B.Cu") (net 8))
 (segment (start 150 98) (end 149.57 97.57) (width 1) (layer "F.Cu") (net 14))
 (segment (start 108 68.88) (end 108 71.42) (width 1) (layer "F.Cu") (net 14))
 (segment (start 149.57 97.57) (end 146.5 97.57) (width 1) (layer "F.Cu") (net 14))
 (segment (start 108 71.42) (end 120.35 71.42) (width 1) (layer "F.Cu") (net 14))
 (segment (start 120.35 71.42) (end 146.5 97.57) (width 1) (layer "F.Cu") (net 14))
 (segment (start 134.5 100) (end 135.5 100) (width 0.6) (layer "F.Cu") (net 3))
 (segment (start 135.5 100) (end 135.61 100.11) (width 0.6) (layer "F.Cu") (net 3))
 (segment (start 108 81.58) (end 116.08 81.58) (width 1) (layer "F.Cu") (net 3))
 (segment (start 116.08 81.58) (end 134.5 100) (width 1) (layer "F.Cu") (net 3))
 (segment (start 135.61 100.11) (end 137.2 100.11) (width 0.6) (layer "F.Cu") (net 3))
 (segment (start 137.2 96.7) (end 137.2 97.57) (width 1) (layer "F.Cu") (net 1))
 (segment (start 141.07 97.57) (end 142.34 98.84) (width 0.6) (layer "F.Cu") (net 1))
 (segment (start 142.34 98.84) (end 146.5 98.84) (width 0.6) (layer "F.Cu") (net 1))
 (segment (start 137.2 97.57) (end 141.07 97.57) (width 0.6) (layer "F.Cu") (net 1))
 (segment (start 114.46 73.96) (end 137.2 96.7) (width 1) (layer "F.Cu") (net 1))
 (segment (start 108 73.96) (end 114.46 73.96) (width 1) (layer "F.Cu") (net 1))
 (segment (start 108 89.2) (end 115.7 89.2) (width 1) (layer "F.Cu") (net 7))
 (segment (start 115.7 89.2) (end 134 107.5) (width 1) (layer "F.Cu") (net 7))
 (segment (start 134.23 107.73) (end 137.2 107.73) (width 0.6) (layer "F.Cu") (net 7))
 (segment (start 134 107.5) (end 134.23 107.73) (width 0.6) (layer "F.Cu") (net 7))
 (segment (start 144.5 101.085001) (end 145.475001 100.11) (width 0.6) (layer "F.Cu") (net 12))
 (segment (start 144.5 101.5) (end 144.5 101.085001) (width 0.6) (layer "F.Cu") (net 12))
 (segment (start 139.254107 109.177131) (end 108.431238 140) (width 1) (layer "F.Cu") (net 12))
 (segment (start 145.475001 100.11) (end 146.5 100.11) (width 0.6) (layer "F.Cu") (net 12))
 (segment (start 108.431238 140) (end 108 140) (width 1) (layer "F.Cu") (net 12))
 (segment (start 139.484925 101.5) (end 139.254107 101.730818) (width 1) (layer "F.Cu") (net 12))
 (segment (start 146.5 102.65) (end 145.475001 102.65) (width 0.6) (layer "F.Cu") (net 12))
 (segment (start 144.5 101.674999) (end 144.5 101.5) (width 0.6) (layer "F.Cu") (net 12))
 (segment (start 145.475001 102.65) (end 144.5 101.674999) (width 0.6) (layer "F.Cu") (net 12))
 (segment (start 139.254107 101.730818) (end 139.254107 109.177131) (width 1) (layer "F.Cu") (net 12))
 (segment (start 144.5 101.5) (end 139.484925 101.5) (width 1) (layer "F.Cu") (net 12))
 (segment (start 135 105) (end 136.46 106.46) (width 0.6) (layer "F.Cu") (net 5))
 (segment (start 134 105) (end 135 105) (width 1) (layer "F.Cu") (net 5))
 (segment (start 135 105) (end 135 104.5) (width 0.6) (layer "F.Cu") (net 5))
 (segment (start 136.46 106.46) (end 137.2 106.46) (width 0.6) (layer "F.Cu") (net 5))
 (segment (start 135 104.5) (end 135.58 103.92) (width 0.6) (layer "F.Cu") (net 5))
 (segment (start 135.58 103.92) (end 137.2 103.92) (width 0.6) (layer "F.Cu") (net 5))
 (via (at 134 105) (size 0.6) (drill 0.3) (layers "F.Cu" "B.Cu") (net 5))
 (segment (start 131.4 107.6) (end 134 105) (width 1) (layer "B.Cu") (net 5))
 (segment (start 159.4 141.905) (end 131.4 141.905) (width 1) (layer "B.Cu") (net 5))
 (segment (start 131.4 141.905) (end 131.4 107.6) (width 1) (layer "B.Cu") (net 5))
 (segment (start 201.058 127.058) (end 201.058 123.047) (width 1) (layer "B.Cu") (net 15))
 (segment (start 201.5 129.5) (end 201.5 127.5) (width 1) (layer "B.Cu") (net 15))
 (segment (start 201.5 127.5) (end 201.058 127.058) (width 1) (layer "B.Cu") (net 15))
 (segment (start 150.75 134.855) (end 196.145 134.855) (width 1) (layer "B.Cu") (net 15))
 (segment (start 196.145 134.855) (end 201.5 129.5) (width 1) (layer "B.Cu") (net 15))
 (segment (start 201.058 123.047) (end 202.48 121.625) (width 1) (layer "B.Cu") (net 15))
 (segment (start 148.95 136.655) (end 150.75 134.855) (width 1) (layer "B.Cu") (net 15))
 (segment (start 139.5 100) (end 139.5 99) (width 1) (layer "F.Cu") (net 2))
 (segment (start 139.5 99) (end 139.34 98.84) (width 0.6) (layer "F.Cu") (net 2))
 (segment (start 139.34 98.84) (end 137.2 98.84) (width 0.6) (layer "F.Cu") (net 2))
 (segment (start 138.12 101.38) (end 139.5 100) (width 0.6) (layer "F.Cu") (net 2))
 (segment (start 137.2 101.38) (end 138.12 101.38) (width 0.6) (layer "F.Cu") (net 2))
 (via (at 139.5 100) (size 0.6) (drill 0.3) (layers "F.Cu" "B.Cu") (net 2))
 (segment (start 140.454107 100.954107) (end 139.5 100) (width 1) (layer "B.Cu") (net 2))
 (segment (start 140.454107 131.200893) (end 140.454107 100.954107) (width 1) (layer "B.Cu") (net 2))
 (segment (start 134.95 136.705) (end 140.454107 131.200893) (width 1) (layer "B.Cu") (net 2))
 (segment (start 158.625 119.125) (end 148.5 109) (width 1) (layer "F.Cu") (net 9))
 (segment (start 199.98 119.125) (end 158.625 119.125) (width 1) (layer "F.Cu") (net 9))
 (segment (start 148.5 109) (end 146.5 109) (width 0.6) (layer "F.Cu") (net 9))
 (segment (start 205 122.218841) (end 201.906159 119.125) (width 0.8) (layer "B.Cu") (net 9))
 (segment (start 199.98 140.635) (end 201.182081 140.635) (width 0.8) (layer "B.Cu") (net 9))
 (segment (start 201.906159 119.125) (end 199.98 119.125) (width 0.8) (layer "B.Cu") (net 9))
 (segment (start 201.182081 140.635) (end 205 136.817081) (width 0.8) (layer "B.Cu") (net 9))
 (segment (start 205 136.817081) (end 205 122.218841) (width 0.8) (layer "B.Cu") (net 9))
 (segment (start 203.982 113.482) (end 192 101.5) (width 1) (layer "F.Cu") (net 13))
 (segment (start 148.5 101.5) (end 146.62 101.5) (width 0.6) (layer "F.Cu") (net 13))
 (segment (start 201.946159 128.61) (end 204 130.663841) (width 0.8) (layer "F.Cu") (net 13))
 (segment (start 192 101.5) (end 148.5 101.5) (width 1) (layer "F.Cu") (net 13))
 (segment (start 204 134.075) (end 199.98 138.095) (width 0.8) (layer "F.Cu") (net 13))
 (segment (start 146.62 101.5) (end 146.5 101.38) (width 0.6) (layer "F.Cu") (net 13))
 (segment (start 202.087581 128.61) (end 203.982 126.715581) (width 1) (layer "F.Cu") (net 13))
 (segment (start 200.02 128.61) (end 202.087581 128.61) (width 1) (layer "F.Cu") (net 13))
 (segment (start 203.982 126.715581) (end 203.982 113.482) (width 1) (layer "F.Cu") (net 13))
 (segment (start 204 130.663841) (end 204 134.075) (width 0.8) (layer "F.Cu") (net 13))
 (segment (start 200.02 128.61) (end 201.946159 128.61) (width 0.8) (layer "F.Cu") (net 13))
 (segment (start 196.975 136.655) (end 202.52 131.11) (width 1) (layer "F.Cu") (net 16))
 (segment (start 162.95 136.655) (end 196.975 136.655) (width 1) (layer "F.Cu") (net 16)))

